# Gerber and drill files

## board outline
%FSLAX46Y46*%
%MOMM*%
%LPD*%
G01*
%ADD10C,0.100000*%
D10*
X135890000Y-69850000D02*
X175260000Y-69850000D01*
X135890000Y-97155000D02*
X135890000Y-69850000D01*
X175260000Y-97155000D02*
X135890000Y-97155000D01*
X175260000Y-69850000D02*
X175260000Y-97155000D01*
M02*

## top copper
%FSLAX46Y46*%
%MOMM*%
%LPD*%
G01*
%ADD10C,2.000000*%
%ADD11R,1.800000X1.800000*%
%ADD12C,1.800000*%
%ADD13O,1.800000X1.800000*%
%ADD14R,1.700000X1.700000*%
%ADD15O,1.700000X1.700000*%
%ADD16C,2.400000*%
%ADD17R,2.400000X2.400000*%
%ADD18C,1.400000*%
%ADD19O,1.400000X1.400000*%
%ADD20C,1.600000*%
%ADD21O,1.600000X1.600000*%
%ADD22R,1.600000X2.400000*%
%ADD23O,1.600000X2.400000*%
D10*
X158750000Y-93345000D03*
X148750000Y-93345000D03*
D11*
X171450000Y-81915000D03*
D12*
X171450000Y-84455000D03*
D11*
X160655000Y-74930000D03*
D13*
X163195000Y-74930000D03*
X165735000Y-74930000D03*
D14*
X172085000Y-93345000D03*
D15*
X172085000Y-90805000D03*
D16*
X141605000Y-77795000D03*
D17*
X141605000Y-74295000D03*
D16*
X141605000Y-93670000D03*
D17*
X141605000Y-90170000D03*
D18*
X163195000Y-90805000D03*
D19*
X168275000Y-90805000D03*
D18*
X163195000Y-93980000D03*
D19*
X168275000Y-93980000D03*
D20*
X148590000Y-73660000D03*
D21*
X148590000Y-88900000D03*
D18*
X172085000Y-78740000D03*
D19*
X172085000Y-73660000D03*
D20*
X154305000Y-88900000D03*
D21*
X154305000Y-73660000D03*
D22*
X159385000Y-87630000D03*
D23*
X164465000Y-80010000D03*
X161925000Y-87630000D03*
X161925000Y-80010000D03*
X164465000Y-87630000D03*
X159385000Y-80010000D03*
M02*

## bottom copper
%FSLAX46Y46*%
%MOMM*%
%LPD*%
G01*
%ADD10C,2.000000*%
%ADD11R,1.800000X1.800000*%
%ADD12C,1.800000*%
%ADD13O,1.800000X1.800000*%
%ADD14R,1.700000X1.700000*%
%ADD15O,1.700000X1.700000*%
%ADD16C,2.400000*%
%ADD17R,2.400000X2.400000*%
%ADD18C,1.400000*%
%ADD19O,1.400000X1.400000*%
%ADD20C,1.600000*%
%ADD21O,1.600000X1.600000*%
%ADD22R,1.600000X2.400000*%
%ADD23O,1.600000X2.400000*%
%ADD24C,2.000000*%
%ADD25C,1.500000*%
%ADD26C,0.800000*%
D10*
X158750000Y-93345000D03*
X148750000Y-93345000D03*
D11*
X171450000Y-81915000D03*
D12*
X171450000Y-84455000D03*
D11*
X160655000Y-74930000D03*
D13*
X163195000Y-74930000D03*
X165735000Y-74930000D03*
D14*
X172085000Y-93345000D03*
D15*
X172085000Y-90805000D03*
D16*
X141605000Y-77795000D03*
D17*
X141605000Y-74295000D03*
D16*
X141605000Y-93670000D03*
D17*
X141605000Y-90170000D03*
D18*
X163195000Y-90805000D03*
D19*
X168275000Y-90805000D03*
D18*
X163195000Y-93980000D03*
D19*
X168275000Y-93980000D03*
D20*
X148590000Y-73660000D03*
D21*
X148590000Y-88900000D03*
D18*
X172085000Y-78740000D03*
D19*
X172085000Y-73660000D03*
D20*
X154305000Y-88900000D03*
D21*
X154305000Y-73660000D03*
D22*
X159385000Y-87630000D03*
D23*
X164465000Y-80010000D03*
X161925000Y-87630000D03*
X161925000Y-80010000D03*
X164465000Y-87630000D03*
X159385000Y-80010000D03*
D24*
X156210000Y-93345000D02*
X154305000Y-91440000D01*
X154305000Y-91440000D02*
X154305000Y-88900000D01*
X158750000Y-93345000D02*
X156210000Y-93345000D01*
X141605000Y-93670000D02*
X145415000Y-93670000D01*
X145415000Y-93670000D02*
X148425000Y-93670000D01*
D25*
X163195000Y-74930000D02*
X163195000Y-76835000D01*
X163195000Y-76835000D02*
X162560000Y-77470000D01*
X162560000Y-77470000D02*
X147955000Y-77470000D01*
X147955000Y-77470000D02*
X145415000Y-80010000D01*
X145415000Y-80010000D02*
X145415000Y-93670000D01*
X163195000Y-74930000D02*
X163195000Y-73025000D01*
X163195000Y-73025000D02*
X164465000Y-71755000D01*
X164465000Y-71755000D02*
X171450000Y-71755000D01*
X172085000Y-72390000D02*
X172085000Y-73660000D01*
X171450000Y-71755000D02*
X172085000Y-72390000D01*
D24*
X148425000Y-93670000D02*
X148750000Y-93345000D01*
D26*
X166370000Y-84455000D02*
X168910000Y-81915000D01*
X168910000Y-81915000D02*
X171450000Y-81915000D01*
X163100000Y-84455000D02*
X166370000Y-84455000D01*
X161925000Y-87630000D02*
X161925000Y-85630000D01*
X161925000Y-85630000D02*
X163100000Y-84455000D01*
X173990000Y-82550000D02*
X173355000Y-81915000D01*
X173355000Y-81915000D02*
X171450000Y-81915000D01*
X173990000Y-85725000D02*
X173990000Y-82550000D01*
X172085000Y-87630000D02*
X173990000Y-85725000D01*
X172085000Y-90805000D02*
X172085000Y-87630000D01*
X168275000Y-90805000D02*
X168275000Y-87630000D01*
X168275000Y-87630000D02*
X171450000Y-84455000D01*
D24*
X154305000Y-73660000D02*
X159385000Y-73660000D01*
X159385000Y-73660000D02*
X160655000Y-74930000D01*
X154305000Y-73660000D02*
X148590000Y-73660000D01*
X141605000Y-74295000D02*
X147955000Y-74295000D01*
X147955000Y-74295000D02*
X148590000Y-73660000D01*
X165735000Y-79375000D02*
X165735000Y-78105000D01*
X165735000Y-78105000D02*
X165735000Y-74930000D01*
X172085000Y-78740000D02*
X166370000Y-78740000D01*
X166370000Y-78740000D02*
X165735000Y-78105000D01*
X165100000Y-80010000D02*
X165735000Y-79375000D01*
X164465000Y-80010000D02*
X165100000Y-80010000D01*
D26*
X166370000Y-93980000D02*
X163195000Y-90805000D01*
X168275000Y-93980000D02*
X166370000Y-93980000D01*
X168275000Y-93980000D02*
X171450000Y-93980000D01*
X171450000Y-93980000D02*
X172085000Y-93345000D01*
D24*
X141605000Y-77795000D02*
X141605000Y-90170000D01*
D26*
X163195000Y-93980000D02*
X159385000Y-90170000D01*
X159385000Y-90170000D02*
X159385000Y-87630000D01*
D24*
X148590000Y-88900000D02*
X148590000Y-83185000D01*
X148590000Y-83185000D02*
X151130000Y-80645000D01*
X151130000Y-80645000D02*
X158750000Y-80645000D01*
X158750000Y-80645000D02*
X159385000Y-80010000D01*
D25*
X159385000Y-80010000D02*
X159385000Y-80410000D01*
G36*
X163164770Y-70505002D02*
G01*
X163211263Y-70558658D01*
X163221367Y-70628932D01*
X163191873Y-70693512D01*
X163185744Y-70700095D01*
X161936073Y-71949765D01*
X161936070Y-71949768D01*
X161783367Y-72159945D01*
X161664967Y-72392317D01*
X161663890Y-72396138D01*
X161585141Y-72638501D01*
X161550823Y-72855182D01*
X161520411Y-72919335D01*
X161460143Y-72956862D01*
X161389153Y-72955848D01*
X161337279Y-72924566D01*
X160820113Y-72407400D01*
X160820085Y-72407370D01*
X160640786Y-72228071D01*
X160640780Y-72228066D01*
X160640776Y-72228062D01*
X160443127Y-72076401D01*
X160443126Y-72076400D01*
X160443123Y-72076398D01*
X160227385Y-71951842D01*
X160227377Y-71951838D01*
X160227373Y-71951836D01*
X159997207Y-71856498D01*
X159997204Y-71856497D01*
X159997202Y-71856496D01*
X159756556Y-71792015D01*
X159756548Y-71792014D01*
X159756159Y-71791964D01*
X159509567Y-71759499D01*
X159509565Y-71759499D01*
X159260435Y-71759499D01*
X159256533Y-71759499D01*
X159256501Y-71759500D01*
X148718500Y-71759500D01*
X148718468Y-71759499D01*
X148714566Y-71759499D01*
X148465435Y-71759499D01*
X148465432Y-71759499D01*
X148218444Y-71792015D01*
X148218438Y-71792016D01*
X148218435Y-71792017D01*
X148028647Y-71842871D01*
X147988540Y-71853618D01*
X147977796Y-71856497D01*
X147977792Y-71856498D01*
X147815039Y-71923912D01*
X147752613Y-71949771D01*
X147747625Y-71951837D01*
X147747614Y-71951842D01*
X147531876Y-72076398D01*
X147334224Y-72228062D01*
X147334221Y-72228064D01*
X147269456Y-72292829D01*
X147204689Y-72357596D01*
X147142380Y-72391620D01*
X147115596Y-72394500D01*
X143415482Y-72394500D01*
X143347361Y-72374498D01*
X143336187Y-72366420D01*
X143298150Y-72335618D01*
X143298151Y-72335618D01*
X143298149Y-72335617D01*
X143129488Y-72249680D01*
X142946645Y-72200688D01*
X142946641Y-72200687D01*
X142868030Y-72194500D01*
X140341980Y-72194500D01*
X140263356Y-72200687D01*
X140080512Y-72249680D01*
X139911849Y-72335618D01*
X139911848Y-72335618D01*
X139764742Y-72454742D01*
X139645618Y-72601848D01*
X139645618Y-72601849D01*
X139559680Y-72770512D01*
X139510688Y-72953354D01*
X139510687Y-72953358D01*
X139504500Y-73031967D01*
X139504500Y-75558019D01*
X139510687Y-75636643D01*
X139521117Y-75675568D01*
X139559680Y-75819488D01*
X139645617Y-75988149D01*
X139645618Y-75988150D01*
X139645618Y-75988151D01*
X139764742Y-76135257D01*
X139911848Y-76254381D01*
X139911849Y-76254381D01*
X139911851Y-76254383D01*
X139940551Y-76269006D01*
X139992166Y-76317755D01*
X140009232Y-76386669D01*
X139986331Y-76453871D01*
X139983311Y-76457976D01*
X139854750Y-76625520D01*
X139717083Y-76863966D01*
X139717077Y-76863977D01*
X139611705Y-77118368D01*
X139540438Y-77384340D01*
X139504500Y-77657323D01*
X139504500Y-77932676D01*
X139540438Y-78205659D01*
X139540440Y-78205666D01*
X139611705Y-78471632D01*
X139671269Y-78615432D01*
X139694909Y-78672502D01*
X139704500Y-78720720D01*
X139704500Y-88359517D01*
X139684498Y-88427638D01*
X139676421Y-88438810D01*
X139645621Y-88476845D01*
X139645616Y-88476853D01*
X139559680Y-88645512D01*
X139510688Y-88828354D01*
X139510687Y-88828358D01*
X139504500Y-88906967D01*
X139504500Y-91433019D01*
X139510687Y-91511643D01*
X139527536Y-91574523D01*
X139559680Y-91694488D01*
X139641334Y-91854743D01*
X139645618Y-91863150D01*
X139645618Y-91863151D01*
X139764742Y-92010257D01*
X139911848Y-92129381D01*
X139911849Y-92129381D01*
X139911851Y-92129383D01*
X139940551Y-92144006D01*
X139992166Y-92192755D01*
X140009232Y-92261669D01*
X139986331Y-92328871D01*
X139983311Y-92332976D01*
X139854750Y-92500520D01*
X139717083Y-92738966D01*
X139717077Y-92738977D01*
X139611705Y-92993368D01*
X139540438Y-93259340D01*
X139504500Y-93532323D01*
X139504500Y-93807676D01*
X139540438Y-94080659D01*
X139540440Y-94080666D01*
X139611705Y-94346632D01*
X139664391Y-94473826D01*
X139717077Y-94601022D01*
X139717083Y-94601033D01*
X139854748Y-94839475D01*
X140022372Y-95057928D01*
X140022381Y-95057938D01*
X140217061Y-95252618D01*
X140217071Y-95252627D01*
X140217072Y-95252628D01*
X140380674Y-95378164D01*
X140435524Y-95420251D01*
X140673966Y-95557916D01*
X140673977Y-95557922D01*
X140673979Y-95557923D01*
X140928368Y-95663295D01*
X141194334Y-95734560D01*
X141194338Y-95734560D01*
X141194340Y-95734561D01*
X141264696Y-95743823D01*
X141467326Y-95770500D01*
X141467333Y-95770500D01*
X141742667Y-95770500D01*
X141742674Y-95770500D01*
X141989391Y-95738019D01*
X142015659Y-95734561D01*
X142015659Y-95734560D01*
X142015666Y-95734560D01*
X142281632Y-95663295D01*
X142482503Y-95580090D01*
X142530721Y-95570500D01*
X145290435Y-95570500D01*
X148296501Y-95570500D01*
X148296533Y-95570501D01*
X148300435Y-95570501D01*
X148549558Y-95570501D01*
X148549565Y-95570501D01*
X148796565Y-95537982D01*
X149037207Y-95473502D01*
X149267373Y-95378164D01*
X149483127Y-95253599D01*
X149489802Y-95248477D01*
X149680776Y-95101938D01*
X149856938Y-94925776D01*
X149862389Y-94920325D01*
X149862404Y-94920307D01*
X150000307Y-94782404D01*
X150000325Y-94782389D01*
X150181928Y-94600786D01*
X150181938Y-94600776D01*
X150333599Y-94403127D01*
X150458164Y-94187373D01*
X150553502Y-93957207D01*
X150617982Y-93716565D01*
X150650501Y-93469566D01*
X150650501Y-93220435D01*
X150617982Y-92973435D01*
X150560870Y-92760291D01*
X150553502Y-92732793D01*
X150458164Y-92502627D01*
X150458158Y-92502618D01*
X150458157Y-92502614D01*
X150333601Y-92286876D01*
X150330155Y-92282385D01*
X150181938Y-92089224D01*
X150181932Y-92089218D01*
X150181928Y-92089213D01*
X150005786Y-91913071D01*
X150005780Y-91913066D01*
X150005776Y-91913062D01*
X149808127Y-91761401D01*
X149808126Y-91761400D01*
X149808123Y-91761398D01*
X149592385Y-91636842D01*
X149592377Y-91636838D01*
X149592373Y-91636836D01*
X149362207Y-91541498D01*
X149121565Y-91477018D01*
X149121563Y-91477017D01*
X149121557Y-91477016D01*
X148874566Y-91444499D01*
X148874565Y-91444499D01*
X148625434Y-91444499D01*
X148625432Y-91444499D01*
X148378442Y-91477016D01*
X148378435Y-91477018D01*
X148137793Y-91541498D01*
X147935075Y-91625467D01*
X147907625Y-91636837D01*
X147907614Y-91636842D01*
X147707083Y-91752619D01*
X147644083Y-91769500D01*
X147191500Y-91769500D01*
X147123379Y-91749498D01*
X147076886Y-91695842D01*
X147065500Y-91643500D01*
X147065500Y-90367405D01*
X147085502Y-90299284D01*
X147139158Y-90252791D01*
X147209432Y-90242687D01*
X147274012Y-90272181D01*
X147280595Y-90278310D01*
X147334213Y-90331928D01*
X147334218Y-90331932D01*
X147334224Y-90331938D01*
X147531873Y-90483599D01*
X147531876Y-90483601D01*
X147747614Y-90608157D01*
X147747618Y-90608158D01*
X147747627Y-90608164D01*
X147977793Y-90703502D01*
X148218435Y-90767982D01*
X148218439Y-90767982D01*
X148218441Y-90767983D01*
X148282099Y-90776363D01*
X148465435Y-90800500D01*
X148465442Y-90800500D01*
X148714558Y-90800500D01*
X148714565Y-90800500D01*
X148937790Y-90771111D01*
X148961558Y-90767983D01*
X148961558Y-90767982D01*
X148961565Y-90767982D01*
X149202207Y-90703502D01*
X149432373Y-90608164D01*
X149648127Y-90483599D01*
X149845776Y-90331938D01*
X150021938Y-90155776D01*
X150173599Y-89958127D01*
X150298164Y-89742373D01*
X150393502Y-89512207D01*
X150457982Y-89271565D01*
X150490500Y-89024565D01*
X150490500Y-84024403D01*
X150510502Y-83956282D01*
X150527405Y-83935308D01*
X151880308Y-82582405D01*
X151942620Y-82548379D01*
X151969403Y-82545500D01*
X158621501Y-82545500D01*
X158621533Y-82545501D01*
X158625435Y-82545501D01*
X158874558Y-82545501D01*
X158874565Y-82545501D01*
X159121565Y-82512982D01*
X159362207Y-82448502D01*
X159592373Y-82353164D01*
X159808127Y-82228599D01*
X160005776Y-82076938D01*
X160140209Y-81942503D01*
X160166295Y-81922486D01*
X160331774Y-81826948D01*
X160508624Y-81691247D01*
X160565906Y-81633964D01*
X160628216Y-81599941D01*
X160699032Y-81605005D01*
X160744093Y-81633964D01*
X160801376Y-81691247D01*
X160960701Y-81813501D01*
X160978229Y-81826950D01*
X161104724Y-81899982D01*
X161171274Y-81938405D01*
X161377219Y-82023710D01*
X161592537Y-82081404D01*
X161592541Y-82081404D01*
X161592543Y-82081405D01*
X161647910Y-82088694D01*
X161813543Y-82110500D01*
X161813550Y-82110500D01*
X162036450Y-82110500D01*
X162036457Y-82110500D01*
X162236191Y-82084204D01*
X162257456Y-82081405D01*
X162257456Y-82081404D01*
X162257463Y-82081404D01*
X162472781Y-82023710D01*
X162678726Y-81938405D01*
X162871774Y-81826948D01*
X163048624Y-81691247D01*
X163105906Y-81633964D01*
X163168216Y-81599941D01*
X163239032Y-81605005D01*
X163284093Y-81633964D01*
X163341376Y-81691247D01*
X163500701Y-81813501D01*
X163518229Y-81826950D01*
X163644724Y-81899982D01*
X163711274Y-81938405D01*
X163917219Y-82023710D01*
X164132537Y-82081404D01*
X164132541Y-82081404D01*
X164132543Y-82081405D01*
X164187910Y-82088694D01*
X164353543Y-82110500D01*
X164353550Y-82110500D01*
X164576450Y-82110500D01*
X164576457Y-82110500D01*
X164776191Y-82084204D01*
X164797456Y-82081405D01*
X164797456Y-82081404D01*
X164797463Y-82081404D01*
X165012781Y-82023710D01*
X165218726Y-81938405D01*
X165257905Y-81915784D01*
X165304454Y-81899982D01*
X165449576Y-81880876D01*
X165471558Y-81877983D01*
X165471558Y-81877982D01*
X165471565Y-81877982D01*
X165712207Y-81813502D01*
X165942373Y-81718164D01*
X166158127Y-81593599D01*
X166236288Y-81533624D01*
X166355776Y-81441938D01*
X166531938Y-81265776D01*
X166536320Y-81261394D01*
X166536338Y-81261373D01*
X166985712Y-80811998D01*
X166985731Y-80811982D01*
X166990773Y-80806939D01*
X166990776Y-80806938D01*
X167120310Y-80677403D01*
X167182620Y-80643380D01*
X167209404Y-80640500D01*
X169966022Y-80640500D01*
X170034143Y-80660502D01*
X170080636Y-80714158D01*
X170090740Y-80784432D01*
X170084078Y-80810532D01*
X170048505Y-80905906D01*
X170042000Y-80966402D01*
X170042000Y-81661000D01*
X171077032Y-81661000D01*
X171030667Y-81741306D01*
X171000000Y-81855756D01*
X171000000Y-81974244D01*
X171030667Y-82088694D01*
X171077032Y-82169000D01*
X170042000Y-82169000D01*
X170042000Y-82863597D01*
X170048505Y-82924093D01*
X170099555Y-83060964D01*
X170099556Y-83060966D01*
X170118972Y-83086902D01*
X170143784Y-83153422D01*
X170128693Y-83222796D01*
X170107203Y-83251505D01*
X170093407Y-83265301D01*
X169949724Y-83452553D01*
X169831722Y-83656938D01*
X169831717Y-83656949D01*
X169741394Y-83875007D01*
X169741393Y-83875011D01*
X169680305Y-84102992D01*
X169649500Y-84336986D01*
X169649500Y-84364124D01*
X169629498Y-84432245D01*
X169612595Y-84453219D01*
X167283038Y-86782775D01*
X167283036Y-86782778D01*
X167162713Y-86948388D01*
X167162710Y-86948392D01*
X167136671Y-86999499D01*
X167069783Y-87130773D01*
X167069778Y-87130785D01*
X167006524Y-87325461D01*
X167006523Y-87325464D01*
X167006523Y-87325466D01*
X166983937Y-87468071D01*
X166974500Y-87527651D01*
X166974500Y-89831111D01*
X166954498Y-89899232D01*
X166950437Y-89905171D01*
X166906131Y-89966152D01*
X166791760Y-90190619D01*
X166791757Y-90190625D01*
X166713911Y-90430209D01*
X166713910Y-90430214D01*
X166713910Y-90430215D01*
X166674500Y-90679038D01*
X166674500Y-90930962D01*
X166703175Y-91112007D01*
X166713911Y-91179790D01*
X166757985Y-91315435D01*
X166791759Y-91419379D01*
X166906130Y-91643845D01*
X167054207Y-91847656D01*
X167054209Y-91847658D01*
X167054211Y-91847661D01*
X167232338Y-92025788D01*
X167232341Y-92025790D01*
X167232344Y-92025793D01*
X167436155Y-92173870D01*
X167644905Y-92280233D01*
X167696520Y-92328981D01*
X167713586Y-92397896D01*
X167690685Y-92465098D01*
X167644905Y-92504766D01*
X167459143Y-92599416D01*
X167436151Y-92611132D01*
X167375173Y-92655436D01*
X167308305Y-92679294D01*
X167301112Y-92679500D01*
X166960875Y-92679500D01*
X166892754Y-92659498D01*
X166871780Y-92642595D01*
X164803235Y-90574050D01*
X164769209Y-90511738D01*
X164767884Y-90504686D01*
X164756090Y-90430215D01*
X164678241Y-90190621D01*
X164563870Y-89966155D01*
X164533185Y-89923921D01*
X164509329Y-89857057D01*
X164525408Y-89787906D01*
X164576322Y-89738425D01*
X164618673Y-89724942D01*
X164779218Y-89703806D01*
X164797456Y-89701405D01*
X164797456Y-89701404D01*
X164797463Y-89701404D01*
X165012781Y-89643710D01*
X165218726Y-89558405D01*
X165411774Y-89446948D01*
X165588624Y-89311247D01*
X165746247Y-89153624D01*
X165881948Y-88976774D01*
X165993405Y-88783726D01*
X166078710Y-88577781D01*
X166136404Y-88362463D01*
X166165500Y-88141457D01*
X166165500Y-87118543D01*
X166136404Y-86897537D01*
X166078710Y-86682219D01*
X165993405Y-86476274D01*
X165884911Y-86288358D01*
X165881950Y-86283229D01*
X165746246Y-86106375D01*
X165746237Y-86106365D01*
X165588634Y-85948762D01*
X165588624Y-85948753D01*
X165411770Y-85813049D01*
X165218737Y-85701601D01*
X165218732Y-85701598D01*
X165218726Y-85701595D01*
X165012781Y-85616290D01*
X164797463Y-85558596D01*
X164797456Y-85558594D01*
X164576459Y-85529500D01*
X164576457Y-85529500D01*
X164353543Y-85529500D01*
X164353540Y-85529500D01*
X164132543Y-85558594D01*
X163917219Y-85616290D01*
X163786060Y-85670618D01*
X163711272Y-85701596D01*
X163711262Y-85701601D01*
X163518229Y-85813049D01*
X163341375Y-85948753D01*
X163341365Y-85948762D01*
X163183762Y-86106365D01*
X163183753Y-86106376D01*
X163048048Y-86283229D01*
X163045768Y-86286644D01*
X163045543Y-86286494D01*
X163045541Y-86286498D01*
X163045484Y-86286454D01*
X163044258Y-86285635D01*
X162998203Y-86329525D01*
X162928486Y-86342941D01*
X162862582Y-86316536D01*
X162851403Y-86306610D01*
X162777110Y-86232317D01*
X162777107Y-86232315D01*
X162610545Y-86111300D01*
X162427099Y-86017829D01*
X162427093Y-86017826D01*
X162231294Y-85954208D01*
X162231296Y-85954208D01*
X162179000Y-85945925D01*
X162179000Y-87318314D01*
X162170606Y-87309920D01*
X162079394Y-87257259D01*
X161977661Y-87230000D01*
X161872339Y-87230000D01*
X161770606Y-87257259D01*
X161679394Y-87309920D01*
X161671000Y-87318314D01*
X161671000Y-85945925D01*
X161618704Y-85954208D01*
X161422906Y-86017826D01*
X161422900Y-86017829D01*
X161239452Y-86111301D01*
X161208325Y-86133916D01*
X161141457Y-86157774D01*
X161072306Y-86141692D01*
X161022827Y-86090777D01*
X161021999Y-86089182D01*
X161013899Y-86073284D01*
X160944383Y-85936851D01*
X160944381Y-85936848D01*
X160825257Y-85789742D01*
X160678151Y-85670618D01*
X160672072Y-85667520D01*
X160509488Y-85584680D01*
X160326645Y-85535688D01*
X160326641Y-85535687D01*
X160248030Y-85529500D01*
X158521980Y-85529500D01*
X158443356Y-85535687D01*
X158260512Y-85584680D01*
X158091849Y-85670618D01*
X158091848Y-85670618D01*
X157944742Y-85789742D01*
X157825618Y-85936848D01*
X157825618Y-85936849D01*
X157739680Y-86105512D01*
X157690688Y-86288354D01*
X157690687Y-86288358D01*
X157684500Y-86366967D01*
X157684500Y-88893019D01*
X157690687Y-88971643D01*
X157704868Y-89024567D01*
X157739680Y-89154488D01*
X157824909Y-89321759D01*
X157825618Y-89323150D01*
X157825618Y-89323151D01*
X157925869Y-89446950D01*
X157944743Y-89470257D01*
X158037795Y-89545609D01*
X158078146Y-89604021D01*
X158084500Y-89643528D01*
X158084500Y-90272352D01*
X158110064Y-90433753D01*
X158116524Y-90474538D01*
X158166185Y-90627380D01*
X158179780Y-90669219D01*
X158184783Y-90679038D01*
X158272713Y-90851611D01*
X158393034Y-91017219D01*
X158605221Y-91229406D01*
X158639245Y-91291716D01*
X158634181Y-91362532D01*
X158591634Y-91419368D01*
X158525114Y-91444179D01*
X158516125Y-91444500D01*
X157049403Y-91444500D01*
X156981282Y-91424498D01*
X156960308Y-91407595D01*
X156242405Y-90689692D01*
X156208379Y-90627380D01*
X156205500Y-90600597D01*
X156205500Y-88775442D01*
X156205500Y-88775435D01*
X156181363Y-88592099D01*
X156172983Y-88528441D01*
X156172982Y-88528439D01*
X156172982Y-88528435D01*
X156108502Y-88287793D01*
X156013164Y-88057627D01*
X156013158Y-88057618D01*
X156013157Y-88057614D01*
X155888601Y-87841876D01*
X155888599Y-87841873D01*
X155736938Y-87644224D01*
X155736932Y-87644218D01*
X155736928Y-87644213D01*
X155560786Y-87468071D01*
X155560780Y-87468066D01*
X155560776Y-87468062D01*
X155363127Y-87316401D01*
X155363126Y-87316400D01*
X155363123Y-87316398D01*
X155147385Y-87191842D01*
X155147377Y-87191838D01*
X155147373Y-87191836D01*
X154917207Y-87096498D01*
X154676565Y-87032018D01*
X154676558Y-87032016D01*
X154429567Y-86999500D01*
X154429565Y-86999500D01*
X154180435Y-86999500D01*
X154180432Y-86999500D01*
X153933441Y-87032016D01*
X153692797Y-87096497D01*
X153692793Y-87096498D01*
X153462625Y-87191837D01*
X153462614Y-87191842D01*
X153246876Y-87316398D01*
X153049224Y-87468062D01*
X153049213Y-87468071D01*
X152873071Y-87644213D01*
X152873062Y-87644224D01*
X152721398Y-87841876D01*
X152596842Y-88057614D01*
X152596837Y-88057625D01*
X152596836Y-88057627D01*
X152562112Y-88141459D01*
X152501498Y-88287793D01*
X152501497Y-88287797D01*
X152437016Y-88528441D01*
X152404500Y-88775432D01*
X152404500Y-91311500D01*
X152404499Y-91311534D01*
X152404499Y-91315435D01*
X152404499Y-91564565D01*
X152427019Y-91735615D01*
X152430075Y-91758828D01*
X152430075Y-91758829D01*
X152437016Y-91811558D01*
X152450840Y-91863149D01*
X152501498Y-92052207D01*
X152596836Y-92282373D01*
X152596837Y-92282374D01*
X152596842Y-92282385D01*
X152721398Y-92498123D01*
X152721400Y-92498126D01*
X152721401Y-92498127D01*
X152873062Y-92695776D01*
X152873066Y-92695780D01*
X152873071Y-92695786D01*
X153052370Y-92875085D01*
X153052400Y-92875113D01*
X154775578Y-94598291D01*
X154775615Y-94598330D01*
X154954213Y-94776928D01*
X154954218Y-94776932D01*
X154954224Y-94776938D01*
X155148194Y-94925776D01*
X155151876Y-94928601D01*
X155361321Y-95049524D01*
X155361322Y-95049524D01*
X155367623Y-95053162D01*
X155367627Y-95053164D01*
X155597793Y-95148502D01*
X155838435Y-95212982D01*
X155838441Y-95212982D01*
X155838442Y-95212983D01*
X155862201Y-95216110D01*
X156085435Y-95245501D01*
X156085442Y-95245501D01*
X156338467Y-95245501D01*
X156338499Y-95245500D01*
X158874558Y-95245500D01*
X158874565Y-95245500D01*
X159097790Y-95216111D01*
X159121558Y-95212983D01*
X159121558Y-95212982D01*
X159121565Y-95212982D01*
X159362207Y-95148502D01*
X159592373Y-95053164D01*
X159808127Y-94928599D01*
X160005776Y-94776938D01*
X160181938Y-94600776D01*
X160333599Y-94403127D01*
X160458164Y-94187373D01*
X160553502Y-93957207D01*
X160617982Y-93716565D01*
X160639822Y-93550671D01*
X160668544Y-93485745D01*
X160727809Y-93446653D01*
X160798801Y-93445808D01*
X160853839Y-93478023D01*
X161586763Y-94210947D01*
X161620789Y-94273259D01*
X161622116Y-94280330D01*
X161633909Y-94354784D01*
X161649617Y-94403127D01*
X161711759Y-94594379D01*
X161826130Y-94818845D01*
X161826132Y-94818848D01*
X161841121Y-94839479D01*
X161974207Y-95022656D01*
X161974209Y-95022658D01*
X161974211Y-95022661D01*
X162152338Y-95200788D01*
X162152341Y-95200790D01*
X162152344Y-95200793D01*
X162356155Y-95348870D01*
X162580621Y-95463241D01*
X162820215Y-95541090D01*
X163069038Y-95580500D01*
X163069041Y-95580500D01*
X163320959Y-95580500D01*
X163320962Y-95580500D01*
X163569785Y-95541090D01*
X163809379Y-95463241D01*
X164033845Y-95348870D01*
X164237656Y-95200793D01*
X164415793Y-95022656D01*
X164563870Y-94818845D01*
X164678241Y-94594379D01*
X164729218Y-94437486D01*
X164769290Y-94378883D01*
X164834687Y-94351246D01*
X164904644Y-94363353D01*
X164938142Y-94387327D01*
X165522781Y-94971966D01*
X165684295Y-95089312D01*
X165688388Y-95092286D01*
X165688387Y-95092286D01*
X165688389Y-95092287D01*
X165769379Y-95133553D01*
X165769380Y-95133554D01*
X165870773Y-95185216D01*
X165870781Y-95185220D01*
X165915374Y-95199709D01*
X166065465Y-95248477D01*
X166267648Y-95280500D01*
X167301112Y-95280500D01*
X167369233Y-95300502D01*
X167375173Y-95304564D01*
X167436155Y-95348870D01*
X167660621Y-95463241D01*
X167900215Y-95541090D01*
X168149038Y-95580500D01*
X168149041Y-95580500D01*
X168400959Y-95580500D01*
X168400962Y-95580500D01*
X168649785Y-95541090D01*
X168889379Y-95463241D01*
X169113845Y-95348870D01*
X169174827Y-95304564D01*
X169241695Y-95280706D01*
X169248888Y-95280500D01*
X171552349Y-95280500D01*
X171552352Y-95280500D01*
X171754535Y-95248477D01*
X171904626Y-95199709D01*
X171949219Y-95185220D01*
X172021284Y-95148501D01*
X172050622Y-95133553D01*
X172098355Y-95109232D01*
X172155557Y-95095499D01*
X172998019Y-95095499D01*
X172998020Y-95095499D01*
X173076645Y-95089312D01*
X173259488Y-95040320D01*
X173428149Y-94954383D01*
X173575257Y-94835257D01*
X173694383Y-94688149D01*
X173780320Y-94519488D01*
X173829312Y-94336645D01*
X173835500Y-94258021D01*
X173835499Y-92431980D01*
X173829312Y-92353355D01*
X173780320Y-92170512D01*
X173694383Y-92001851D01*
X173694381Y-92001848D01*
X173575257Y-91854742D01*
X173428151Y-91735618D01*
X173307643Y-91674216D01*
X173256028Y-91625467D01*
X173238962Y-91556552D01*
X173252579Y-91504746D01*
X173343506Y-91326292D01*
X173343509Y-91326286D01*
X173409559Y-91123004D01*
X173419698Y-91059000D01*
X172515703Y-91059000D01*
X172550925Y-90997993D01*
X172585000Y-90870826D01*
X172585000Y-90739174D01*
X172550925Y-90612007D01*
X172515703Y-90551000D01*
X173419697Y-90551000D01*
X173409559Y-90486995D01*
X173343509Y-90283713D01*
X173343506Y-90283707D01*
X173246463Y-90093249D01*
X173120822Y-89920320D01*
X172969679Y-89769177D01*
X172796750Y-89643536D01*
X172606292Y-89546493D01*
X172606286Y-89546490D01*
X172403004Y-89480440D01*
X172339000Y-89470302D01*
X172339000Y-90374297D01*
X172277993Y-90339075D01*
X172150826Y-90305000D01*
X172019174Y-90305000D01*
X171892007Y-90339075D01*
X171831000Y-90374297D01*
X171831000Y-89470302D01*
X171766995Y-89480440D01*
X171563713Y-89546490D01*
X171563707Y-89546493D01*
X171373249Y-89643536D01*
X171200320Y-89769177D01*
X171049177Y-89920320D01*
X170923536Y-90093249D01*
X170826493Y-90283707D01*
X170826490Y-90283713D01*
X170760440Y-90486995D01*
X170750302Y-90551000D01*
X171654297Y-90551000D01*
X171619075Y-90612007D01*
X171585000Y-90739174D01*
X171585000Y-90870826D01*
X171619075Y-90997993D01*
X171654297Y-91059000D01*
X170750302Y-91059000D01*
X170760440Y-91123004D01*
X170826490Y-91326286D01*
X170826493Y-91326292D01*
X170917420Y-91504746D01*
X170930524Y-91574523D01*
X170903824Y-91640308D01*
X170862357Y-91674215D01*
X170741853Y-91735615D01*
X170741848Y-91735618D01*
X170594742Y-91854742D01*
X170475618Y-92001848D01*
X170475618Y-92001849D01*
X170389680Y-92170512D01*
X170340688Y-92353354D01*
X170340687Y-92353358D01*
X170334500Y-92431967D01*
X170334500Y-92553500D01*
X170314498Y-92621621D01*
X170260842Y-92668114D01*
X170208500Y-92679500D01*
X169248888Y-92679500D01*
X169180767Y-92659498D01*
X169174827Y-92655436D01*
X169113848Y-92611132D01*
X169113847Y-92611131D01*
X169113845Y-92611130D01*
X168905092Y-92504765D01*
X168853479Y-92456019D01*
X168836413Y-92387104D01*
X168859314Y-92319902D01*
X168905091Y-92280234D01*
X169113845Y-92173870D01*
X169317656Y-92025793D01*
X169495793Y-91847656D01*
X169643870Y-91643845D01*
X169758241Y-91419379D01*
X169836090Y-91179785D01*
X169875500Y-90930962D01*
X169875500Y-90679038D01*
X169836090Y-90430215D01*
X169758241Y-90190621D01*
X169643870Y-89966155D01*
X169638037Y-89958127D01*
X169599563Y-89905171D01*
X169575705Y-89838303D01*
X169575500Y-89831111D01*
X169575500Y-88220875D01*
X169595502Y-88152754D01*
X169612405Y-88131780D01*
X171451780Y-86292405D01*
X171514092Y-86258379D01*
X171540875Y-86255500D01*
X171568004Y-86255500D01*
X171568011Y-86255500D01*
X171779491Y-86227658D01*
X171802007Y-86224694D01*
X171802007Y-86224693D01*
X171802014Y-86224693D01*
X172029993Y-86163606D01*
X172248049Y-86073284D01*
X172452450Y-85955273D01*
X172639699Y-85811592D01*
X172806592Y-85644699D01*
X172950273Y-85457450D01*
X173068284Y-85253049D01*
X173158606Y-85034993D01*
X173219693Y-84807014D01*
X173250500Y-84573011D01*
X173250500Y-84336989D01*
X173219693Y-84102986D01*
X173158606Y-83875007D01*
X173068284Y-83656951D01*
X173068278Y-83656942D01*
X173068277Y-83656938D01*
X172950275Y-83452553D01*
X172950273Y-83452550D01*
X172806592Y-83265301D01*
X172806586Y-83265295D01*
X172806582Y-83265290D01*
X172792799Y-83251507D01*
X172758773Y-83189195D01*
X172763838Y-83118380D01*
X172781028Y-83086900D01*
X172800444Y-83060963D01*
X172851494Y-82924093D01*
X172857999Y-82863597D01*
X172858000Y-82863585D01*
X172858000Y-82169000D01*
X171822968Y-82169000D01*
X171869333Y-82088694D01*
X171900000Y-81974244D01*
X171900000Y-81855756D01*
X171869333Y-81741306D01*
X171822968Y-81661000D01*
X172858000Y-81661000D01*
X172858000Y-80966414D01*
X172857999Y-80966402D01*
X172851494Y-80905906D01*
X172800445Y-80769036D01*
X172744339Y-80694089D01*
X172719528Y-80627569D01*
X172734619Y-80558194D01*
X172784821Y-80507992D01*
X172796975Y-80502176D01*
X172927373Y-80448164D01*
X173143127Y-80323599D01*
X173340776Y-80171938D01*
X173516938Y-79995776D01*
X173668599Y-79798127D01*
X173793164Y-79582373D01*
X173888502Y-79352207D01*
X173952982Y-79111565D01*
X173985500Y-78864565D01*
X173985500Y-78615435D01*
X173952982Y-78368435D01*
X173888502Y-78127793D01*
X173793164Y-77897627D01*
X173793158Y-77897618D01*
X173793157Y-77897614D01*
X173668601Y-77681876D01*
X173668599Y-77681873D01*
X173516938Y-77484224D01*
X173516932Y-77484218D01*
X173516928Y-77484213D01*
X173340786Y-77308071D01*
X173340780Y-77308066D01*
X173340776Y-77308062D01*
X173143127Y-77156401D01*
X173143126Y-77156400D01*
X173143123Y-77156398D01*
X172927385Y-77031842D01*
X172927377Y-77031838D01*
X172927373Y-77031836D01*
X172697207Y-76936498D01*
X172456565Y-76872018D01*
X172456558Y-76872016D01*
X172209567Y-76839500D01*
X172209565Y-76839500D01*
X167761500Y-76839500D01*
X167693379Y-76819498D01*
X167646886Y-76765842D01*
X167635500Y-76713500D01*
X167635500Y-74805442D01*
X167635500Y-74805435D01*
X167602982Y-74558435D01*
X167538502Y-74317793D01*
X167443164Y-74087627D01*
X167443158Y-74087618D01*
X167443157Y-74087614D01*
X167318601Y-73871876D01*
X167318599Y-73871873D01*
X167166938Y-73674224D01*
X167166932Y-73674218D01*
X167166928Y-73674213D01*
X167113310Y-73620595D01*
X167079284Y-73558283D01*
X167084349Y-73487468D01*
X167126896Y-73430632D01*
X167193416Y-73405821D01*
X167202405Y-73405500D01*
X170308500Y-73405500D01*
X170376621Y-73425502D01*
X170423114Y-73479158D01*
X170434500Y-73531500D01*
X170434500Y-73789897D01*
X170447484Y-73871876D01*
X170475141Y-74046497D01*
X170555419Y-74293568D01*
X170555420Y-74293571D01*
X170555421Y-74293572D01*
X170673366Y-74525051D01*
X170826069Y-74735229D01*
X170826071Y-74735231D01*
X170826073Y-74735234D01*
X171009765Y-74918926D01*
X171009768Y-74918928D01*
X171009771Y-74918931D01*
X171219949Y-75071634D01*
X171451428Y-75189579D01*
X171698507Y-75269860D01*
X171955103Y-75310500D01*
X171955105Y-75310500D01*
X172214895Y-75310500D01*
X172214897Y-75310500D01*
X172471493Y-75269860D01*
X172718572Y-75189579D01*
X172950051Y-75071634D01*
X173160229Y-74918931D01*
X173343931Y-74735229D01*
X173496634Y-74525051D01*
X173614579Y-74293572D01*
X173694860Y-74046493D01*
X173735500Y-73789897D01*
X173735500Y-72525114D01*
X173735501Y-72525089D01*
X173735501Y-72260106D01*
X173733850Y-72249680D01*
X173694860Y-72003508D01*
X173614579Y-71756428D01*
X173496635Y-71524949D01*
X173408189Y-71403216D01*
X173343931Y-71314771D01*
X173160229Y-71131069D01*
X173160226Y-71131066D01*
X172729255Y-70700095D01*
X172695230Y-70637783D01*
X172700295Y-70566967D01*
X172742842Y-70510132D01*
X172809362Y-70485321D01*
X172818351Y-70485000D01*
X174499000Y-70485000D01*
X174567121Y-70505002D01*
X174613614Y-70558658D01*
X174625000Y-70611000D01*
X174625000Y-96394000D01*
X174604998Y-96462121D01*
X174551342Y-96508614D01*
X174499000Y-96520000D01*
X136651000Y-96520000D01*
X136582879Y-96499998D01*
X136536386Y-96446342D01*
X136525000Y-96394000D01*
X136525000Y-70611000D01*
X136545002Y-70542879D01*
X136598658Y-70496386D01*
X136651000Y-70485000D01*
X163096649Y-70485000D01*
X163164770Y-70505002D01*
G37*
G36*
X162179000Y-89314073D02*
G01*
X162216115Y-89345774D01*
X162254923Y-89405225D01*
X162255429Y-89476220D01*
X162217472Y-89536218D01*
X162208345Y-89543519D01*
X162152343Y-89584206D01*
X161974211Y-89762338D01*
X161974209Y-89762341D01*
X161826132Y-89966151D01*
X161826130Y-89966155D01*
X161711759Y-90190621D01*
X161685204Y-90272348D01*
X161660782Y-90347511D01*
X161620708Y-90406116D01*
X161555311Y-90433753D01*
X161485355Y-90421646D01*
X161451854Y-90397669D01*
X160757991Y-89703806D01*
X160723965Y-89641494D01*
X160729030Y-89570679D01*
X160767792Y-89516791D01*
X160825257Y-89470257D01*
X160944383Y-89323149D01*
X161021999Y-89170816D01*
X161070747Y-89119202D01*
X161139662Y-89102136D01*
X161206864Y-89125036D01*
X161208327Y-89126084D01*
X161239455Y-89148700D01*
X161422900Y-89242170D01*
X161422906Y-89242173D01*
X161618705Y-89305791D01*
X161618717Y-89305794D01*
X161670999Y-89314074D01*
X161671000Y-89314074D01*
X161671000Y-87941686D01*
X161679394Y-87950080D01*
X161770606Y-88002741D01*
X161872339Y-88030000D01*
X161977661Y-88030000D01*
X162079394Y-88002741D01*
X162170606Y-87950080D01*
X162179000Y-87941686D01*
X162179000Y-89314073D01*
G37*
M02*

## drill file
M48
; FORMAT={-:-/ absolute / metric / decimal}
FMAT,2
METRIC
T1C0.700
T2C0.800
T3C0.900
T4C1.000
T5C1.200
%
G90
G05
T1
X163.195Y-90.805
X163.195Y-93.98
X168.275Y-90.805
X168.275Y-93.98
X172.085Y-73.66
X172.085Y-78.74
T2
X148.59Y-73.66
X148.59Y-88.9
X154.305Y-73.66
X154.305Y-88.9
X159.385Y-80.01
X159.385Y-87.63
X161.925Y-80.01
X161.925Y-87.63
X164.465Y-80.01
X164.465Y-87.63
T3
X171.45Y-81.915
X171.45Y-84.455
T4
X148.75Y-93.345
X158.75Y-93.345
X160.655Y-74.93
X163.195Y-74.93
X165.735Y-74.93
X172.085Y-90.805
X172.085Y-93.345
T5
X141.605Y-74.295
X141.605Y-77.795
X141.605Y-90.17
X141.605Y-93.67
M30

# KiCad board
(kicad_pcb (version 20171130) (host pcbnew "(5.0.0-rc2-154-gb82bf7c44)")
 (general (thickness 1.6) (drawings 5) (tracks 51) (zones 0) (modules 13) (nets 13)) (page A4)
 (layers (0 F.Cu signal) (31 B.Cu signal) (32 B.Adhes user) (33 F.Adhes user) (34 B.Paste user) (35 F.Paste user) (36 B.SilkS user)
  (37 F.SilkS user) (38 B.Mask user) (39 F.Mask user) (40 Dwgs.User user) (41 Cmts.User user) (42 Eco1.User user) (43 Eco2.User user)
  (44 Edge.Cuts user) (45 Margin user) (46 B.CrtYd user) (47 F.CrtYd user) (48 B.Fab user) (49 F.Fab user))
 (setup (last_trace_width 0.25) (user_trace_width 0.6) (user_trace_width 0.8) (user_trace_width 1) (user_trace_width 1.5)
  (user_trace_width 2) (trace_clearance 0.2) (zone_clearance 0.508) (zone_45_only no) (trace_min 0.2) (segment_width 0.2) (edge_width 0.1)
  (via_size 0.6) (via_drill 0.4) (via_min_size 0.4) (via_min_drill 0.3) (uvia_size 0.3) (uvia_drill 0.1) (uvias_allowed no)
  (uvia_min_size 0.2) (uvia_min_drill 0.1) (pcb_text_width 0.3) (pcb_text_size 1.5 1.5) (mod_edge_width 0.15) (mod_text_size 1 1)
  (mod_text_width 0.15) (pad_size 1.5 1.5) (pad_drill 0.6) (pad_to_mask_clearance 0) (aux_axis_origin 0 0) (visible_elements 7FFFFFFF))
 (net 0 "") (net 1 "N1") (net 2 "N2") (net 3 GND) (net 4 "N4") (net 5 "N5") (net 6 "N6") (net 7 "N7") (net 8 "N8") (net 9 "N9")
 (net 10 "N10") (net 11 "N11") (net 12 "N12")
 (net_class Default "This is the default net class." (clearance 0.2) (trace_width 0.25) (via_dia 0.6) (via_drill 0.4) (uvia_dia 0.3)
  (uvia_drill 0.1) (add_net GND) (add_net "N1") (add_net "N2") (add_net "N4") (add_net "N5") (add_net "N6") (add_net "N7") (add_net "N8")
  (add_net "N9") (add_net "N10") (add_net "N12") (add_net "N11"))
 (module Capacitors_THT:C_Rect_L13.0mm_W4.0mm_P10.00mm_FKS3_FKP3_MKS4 (layer F.Cu) (at 158.75 93.345 180)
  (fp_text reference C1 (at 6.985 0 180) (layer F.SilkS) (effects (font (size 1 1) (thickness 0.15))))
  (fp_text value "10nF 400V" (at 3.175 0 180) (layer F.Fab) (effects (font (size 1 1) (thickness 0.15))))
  (pad 1 thru_hole circle (at 0 0 180) (size 2 2) (drill 1) (layers *.Cu *.Mask) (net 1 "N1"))
  (pad 2 thru_hole circle (at 10 0 180) (size 2 2) (drill 1) (layers *.Cu *.Mask) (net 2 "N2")))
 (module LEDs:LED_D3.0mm (layer F.Cu) (at 171.45 81.915 270)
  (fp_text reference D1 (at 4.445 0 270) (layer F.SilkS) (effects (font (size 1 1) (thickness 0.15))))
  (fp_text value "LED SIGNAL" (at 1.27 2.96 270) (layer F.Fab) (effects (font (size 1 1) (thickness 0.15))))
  (pad 1 thru_hole rect (at 0 0 270) (size 1.8 1.8) (drill 0.9) (layers *.Cu *.Mask) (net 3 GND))
  (pad 2 thru_hole circle (at 2.54 0 270) (size 1.8 1.8) (drill 0.9) (layers *.Cu *.Mask) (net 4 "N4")))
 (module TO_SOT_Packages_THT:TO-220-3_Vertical (layer F.Cu) (at 160.655 74.93)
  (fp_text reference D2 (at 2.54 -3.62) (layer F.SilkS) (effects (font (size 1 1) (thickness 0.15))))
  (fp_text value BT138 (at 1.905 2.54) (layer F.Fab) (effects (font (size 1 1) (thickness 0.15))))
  (pad 1 thru_hole rect (at 0 0) (size 1.8 1.8) (drill 1) (layers *.Cu *.Mask) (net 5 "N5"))
  (pad 2 thru_hole oval (at 2.54 0) (size 1.8 1.8) (drill 1) (layers *.Cu *.Mask) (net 2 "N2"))
  (pad 3 thru_hole oval (at 5.08 0) (size 1.8 1.8) (drill 1) (layers *.Cu *.Mask) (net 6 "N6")))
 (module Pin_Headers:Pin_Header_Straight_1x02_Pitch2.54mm (layer F.Cu) (at 172.085 93.345 180)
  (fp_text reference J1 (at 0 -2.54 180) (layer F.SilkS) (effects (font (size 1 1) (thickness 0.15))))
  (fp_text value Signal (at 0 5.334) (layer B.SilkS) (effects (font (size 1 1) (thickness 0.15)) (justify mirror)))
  (pad 1 thru_hole rect (at 0 0 180) (size 1.7 1.7) (drill 1) (layers *.Cu *.Mask) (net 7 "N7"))
  (pad 2 thru_hole oval (at 0 2.54 180) (size 1.7 1.7) (drill 1) (layers *.Cu *.Mask) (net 3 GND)))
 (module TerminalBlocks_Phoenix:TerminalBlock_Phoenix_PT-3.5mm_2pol (layer F.Cu) (at 141.605 74.295 270)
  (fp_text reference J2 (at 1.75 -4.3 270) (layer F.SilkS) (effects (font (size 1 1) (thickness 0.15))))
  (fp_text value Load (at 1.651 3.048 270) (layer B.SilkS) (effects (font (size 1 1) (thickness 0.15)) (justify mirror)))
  (pad 2 thru_hole circle (at 3.5 0 270) (size 2.4 2.4) (drill 1.2) (layers *.Cu *.Mask) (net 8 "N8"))
  (pad 1 thru_hole rect (at 0 0 270) (size 2.4 2.4) (drill 1.2) (layers *.Cu *.Mask) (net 5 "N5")))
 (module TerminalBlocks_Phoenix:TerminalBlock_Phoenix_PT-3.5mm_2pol (layer F.Cu) (at 141.605 90.17 270)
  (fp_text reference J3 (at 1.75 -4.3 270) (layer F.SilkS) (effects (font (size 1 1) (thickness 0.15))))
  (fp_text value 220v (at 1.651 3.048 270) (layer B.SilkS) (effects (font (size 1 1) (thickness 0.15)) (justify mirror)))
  (pad 2 thru_hole circle (at 3.5 0 270) (size 2.4 2.4) (drill 1.2) (layers *.Cu *.Mask) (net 2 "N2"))
  (pad 1 thru_hole rect (at 0 0 270) (size 2.4 2.4) (drill 1.2) (layers *.Cu *.Mask) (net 8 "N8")))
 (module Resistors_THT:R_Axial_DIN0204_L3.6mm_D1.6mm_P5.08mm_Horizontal (layer F.Cu) (at 163.195 90.805)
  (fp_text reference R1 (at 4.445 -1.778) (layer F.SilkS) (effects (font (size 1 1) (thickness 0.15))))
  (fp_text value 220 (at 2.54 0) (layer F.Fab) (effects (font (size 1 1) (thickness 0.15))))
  (pad 1 thru_hole circle (at 0 0) (size 1.4 1.4) (drill 0.7) (layers *.Cu *.Mask) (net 7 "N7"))
  (pad 2 thru_hole oval (at 5.08 0) (size 1.4 1.4) (drill 0.7) (layers *.Cu *.Mask) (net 4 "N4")))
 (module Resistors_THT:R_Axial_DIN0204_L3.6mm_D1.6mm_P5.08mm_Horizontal (layer F.Cu) (at 163.195 93.98)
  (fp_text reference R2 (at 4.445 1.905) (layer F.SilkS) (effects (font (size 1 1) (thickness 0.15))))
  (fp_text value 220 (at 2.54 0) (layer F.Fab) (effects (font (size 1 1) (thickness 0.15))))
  (pad 1 thru_hole circle (at 0 0) (size 1.4 1.4) (drill 0.7) (layers *.Cu *.Mask) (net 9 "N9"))
  (pad 2 thru_hole oval (at 5.08 0) (size 1.4 1.4) (drill 0.7) (layers *.Cu *.Mask) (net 7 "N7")))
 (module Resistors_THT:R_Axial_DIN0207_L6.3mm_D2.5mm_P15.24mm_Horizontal (layer F.Cu) (at 148.59 73.66 270)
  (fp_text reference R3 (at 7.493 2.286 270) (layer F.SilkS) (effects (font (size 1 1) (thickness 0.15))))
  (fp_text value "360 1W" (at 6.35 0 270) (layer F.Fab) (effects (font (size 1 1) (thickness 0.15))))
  (pad 1 thru_hole circle (at 0 0 270) (size 1.6 1.6) (drill 0.8) (layers *.Cu *.Mask) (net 5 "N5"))
  (pad 2 thru_hole oval (at 15.24 0 270) (size 1.6 1.6) (drill 0.8) (layers *.Cu *.Mask) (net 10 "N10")))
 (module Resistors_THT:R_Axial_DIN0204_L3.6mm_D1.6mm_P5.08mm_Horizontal (layer F.Cu) (at 172.085 78.74 90)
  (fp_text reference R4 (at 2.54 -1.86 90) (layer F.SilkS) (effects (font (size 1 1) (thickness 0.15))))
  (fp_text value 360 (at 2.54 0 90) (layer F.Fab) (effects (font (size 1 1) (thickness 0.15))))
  (pad 1 thru_hole circle (at 0 0 90) (size 1.4 1.4) (drill 0.7) (layers *.Cu *.Mask) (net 6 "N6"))
  (pad 2 thru_hole oval (at 5.08 0 90) (size 1.4 1.4) (drill 0.7) (layers *.Cu *.Mask) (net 2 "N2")))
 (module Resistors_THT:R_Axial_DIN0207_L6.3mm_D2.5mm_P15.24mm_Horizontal (layer F.Cu) (at 154.305 88.9 90)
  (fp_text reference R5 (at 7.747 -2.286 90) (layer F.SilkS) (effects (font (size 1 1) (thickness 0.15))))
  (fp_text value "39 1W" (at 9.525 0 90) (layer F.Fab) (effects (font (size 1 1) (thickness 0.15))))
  (pad 1 thru_hole circle (at 0 0 90) (size 1.6 1.6) (drill 0.8) (layers *.Cu *.Mask) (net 1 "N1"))
  (pad 2 thru_hole oval (at 15.24 0 90) (size 1.6 1.6) (drill 0.8) (layers *.Cu *.Mask) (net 5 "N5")))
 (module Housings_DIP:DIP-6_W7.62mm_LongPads (layer F.Cu) (at 159.385 87.63 90)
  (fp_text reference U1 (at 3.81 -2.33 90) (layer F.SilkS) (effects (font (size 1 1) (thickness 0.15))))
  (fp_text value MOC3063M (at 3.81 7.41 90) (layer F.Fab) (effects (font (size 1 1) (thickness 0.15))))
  (pad 1 thru_hole rect (at 0 0 90) (size 2.4 1.6) (drill 0.8) (layers *.Cu *.Mask) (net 9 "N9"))
  (pad 4 thru_hole oval (at 7.62 5.08 90) (size 2.4 1.6) (drill 0.8) (layers *.Cu *.Mask) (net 6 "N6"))
  (pad 2 thru_hole oval (at 0 2.54 90) (size 2.4 1.6) (drill 0.8) (layers *.Cu *.Mask) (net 3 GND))
  (pad 5 thru_hole oval (at 7.62 2.54 90) (size 2.4 1.6) (drill 0.8) (layers *.Cu *.Mask) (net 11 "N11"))
  (pad 3 thru_hole oval (at 0 5.08 90) (size 2.4 1.6) (drill 0.8) (layers *.Cu *.Mask) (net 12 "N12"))
  (pad 6 thru_hole oval (at 7.62 0 90) (size 2.4 1.6) (drill 0.8) (layers *.Cu *.Mask) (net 10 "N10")))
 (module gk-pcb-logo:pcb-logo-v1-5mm (layer F.Cu) (at 141.605 83.82 270)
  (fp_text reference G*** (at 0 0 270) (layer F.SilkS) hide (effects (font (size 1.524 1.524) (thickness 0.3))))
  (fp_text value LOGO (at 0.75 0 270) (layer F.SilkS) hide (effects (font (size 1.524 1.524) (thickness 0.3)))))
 (gr_line (start 135.89 69.85) (end 175.26 69.85) (layer Edge.Cuts) (width 0.1))
 (gr_line (start 135.89 97.155) (end 135.89 69.85) (layer Edge.Cuts) (width 0.1))
 (gr_line (start 175.26 97.155) (end 135.89 97.155) (layer Edge.Cuts) (width 0.1))
 (gr_line (start 175.26 69.85) (end 175.26 97.155) (layer Edge.Cuts) (width 0.1))
 (segment (start 156.21 93.345) (end 154.305 91.44) (width 2) (layer B.Cu) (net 1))
 (segment (start 154.305 91.44) (end 154.305 88.9) (width 2) (layer B.Cu) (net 1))
 (segment (start 158.75 93.345) (end 156.21 93.345) (width 2) (layer B.Cu) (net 1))
 (segment (start 141.605 93.67) (end 145.415 93.67) (width 2) (layer B.Cu) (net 2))
 (segment (start 145.415 93.67) (end 148.425 93.67) (width 2) (layer B.Cu) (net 2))
 (segment (start 163.195 74.93) (end 163.195 76.835) (width 1.5) (layer B.Cu) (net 2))
 (segment (start 163.195 76.835) (end 162.56 77.47) (width 1.5) (layer B.Cu) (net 2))
 (segment (start 162.56 77.47) (end 147.955 77.47) (width 1.5) (layer B.Cu) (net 2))
 (segment (start 147.955 77.47) (end 145.415 80.01) (width 1.5) (layer B.Cu) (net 2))
 (segment (start 145.415 80.01) (end 145.415 93.67) (width 1.5) (layer B.Cu) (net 2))
 (segment (start 163.195 74.93) (end 163.195 73.025) (width 1.5) (layer B.Cu) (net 2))
 (segment (start 163.195 73.025) (end 164.465 71.755) (width 1.5) (layer B.Cu) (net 2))
 (segment (start 164.465 71.755) (end 171.45 71.755) (width 1.5) (layer B.Cu) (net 2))
 (segment (start 172.085 72.39) (end 172.085 73.66) (width 1.5) (layer B.Cu) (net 2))
 (segment (start 171.45 71.755) (end 172.085 72.39) (width 1.5) (layer B.Cu) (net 2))
 (segment (start 148.425 93.67) (end 148.75 93.345) (width 2) (layer B.Cu) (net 2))
 (segment (start 166.37 84.455) (end 168.91 81.915) (width 0.8) (layer B.Cu) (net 3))
 (segment (start 168.91 81.915) (end 171.45 81.915) (width 0.8) (layer B.Cu) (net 3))
 (segment (start 163.1 84.455) (end 166.37 84.455) (width 0.8) (layer B.Cu) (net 3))
 (segment (start 161.925 87.63) (end 161.925 85.63) (width 0.8) (layer B.Cu) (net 3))
 (segment (start 161.925 85.63) (end 163.1 84.455) (width 0.8) (layer B.Cu) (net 3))
 (segment (start 173.99 82.55) (end 173.355 81.915) (width 0.8) (layer B.Cu) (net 3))
 (segment (start 173.355 81.915) (end 171.45 81.915) (width 0.8) (layer B.Cu) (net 3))
 (segment (start 173.99 85.725) (end 173.99 82.55) (width 0.8) (layer B.Cu) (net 3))
 (segment (start 172.085 87.63) (end 173.99 85.725) (width 0.8) (layer B.Cu) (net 3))
 (segment (start 172.085 90.805) (end 172.085 87.63) (width 0.8) (layer B.Cu) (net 3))
 (segment (start 168.275 90.805) (end 168.275 87.63) (width 0.8) (layer B.Cu) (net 4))
 (segment (start 168.275 87.63) (end 171.45 84.455) (width 0.8) (layer B.Cu) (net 4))
 (segment (start 154.305 73.66) (end 159.385 73.66) (width 2) (layer B.Cu) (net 5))
 (segment (start 159.385 73.66) (end 160.655 74.93) (width 2) (layer B.Cu) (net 5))
 (segment (start 154.305 73.66) (end 148.59 73.66) (width 2) (layer B.Cu) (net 5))
 (segment (start 141.605 74.295) (end 147.955 74.295) (width 2) (layer B.Cu) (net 5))
 (segment (start 147.955 74.295) (end 148.59 73.66) (width 2) (layer B.Cu) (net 5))
 (segment (start 165.735 79.375) (end 165.735 78.105) (width 2) (layer B.Cu) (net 6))
 (segment (start 165.735 78.105) (end 165.735 74.93) (width 2) (layer B.Cu) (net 6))
 (segment (start 172.085 78.74) (end 166.37 78.74) (width 2) (layer B.Cu) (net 6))
 (segment (start 166.37 78.74) (end 165.735 78.105) (width 2) (layer B.Cu) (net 6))
 (segment (start 165.1 80.01) (end 165.735 79.375) (width 2) (layer B.Cu) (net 6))
 (segment (start 164.465 80.01) (end 165.1 80.01) (width 2) (layer B.Cu) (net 6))
 (segment (start 166.37 93.98) (end 163.195 90.805) (width 0.8) (layer B.Cu) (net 7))
 (segment (start 168.275 93.98) (end 166.37 93.98) (width 0.8) (layer B.Cu) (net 7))
 (segment (start 168.275 93.98) (end 171.45 93.98) (width 0.8) (layer B.Cu) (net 7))
 (segment (start 171.45 93.98) (end 172.085 93.345) (width 0.8) (layer B.Cu) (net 7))
 (segment (start 141.605 77.795) (end 141.605 90.17) (width 2) (layer B.Cu) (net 8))
 (segment (start 163.195 93.98) (end 159.385 90.17) (width 0.8) (layer B.Cu) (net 9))
 (segment (start 159.385 90.17) (end 159.385 87.63) (width 0.8) (layer B.Cu) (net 9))
 (segment (start 148.59 88.9) (end 148.59 83.185) (width 2) (layer B.Cu) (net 10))
 (segment (start 148.59 83.185) (end 151.13 80.645) (width 2) (layer B.Cu) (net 10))
 (segment (start 151.13 80.645) (end 158.75 80.645) (width 2) (layer B.Cu) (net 10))
 (segment (start 158.75 80.645) (end 159.385 80.01) (width 2) (layer B.Cu) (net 10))
 (segment (start 159.385 80.01) (end 159.385 80.41) (width 1.5) (layer B.Cu) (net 10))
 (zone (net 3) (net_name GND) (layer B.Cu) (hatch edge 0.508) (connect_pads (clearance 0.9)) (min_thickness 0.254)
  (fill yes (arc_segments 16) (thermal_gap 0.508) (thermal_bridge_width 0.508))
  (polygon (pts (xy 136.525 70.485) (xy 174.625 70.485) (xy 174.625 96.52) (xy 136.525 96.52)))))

